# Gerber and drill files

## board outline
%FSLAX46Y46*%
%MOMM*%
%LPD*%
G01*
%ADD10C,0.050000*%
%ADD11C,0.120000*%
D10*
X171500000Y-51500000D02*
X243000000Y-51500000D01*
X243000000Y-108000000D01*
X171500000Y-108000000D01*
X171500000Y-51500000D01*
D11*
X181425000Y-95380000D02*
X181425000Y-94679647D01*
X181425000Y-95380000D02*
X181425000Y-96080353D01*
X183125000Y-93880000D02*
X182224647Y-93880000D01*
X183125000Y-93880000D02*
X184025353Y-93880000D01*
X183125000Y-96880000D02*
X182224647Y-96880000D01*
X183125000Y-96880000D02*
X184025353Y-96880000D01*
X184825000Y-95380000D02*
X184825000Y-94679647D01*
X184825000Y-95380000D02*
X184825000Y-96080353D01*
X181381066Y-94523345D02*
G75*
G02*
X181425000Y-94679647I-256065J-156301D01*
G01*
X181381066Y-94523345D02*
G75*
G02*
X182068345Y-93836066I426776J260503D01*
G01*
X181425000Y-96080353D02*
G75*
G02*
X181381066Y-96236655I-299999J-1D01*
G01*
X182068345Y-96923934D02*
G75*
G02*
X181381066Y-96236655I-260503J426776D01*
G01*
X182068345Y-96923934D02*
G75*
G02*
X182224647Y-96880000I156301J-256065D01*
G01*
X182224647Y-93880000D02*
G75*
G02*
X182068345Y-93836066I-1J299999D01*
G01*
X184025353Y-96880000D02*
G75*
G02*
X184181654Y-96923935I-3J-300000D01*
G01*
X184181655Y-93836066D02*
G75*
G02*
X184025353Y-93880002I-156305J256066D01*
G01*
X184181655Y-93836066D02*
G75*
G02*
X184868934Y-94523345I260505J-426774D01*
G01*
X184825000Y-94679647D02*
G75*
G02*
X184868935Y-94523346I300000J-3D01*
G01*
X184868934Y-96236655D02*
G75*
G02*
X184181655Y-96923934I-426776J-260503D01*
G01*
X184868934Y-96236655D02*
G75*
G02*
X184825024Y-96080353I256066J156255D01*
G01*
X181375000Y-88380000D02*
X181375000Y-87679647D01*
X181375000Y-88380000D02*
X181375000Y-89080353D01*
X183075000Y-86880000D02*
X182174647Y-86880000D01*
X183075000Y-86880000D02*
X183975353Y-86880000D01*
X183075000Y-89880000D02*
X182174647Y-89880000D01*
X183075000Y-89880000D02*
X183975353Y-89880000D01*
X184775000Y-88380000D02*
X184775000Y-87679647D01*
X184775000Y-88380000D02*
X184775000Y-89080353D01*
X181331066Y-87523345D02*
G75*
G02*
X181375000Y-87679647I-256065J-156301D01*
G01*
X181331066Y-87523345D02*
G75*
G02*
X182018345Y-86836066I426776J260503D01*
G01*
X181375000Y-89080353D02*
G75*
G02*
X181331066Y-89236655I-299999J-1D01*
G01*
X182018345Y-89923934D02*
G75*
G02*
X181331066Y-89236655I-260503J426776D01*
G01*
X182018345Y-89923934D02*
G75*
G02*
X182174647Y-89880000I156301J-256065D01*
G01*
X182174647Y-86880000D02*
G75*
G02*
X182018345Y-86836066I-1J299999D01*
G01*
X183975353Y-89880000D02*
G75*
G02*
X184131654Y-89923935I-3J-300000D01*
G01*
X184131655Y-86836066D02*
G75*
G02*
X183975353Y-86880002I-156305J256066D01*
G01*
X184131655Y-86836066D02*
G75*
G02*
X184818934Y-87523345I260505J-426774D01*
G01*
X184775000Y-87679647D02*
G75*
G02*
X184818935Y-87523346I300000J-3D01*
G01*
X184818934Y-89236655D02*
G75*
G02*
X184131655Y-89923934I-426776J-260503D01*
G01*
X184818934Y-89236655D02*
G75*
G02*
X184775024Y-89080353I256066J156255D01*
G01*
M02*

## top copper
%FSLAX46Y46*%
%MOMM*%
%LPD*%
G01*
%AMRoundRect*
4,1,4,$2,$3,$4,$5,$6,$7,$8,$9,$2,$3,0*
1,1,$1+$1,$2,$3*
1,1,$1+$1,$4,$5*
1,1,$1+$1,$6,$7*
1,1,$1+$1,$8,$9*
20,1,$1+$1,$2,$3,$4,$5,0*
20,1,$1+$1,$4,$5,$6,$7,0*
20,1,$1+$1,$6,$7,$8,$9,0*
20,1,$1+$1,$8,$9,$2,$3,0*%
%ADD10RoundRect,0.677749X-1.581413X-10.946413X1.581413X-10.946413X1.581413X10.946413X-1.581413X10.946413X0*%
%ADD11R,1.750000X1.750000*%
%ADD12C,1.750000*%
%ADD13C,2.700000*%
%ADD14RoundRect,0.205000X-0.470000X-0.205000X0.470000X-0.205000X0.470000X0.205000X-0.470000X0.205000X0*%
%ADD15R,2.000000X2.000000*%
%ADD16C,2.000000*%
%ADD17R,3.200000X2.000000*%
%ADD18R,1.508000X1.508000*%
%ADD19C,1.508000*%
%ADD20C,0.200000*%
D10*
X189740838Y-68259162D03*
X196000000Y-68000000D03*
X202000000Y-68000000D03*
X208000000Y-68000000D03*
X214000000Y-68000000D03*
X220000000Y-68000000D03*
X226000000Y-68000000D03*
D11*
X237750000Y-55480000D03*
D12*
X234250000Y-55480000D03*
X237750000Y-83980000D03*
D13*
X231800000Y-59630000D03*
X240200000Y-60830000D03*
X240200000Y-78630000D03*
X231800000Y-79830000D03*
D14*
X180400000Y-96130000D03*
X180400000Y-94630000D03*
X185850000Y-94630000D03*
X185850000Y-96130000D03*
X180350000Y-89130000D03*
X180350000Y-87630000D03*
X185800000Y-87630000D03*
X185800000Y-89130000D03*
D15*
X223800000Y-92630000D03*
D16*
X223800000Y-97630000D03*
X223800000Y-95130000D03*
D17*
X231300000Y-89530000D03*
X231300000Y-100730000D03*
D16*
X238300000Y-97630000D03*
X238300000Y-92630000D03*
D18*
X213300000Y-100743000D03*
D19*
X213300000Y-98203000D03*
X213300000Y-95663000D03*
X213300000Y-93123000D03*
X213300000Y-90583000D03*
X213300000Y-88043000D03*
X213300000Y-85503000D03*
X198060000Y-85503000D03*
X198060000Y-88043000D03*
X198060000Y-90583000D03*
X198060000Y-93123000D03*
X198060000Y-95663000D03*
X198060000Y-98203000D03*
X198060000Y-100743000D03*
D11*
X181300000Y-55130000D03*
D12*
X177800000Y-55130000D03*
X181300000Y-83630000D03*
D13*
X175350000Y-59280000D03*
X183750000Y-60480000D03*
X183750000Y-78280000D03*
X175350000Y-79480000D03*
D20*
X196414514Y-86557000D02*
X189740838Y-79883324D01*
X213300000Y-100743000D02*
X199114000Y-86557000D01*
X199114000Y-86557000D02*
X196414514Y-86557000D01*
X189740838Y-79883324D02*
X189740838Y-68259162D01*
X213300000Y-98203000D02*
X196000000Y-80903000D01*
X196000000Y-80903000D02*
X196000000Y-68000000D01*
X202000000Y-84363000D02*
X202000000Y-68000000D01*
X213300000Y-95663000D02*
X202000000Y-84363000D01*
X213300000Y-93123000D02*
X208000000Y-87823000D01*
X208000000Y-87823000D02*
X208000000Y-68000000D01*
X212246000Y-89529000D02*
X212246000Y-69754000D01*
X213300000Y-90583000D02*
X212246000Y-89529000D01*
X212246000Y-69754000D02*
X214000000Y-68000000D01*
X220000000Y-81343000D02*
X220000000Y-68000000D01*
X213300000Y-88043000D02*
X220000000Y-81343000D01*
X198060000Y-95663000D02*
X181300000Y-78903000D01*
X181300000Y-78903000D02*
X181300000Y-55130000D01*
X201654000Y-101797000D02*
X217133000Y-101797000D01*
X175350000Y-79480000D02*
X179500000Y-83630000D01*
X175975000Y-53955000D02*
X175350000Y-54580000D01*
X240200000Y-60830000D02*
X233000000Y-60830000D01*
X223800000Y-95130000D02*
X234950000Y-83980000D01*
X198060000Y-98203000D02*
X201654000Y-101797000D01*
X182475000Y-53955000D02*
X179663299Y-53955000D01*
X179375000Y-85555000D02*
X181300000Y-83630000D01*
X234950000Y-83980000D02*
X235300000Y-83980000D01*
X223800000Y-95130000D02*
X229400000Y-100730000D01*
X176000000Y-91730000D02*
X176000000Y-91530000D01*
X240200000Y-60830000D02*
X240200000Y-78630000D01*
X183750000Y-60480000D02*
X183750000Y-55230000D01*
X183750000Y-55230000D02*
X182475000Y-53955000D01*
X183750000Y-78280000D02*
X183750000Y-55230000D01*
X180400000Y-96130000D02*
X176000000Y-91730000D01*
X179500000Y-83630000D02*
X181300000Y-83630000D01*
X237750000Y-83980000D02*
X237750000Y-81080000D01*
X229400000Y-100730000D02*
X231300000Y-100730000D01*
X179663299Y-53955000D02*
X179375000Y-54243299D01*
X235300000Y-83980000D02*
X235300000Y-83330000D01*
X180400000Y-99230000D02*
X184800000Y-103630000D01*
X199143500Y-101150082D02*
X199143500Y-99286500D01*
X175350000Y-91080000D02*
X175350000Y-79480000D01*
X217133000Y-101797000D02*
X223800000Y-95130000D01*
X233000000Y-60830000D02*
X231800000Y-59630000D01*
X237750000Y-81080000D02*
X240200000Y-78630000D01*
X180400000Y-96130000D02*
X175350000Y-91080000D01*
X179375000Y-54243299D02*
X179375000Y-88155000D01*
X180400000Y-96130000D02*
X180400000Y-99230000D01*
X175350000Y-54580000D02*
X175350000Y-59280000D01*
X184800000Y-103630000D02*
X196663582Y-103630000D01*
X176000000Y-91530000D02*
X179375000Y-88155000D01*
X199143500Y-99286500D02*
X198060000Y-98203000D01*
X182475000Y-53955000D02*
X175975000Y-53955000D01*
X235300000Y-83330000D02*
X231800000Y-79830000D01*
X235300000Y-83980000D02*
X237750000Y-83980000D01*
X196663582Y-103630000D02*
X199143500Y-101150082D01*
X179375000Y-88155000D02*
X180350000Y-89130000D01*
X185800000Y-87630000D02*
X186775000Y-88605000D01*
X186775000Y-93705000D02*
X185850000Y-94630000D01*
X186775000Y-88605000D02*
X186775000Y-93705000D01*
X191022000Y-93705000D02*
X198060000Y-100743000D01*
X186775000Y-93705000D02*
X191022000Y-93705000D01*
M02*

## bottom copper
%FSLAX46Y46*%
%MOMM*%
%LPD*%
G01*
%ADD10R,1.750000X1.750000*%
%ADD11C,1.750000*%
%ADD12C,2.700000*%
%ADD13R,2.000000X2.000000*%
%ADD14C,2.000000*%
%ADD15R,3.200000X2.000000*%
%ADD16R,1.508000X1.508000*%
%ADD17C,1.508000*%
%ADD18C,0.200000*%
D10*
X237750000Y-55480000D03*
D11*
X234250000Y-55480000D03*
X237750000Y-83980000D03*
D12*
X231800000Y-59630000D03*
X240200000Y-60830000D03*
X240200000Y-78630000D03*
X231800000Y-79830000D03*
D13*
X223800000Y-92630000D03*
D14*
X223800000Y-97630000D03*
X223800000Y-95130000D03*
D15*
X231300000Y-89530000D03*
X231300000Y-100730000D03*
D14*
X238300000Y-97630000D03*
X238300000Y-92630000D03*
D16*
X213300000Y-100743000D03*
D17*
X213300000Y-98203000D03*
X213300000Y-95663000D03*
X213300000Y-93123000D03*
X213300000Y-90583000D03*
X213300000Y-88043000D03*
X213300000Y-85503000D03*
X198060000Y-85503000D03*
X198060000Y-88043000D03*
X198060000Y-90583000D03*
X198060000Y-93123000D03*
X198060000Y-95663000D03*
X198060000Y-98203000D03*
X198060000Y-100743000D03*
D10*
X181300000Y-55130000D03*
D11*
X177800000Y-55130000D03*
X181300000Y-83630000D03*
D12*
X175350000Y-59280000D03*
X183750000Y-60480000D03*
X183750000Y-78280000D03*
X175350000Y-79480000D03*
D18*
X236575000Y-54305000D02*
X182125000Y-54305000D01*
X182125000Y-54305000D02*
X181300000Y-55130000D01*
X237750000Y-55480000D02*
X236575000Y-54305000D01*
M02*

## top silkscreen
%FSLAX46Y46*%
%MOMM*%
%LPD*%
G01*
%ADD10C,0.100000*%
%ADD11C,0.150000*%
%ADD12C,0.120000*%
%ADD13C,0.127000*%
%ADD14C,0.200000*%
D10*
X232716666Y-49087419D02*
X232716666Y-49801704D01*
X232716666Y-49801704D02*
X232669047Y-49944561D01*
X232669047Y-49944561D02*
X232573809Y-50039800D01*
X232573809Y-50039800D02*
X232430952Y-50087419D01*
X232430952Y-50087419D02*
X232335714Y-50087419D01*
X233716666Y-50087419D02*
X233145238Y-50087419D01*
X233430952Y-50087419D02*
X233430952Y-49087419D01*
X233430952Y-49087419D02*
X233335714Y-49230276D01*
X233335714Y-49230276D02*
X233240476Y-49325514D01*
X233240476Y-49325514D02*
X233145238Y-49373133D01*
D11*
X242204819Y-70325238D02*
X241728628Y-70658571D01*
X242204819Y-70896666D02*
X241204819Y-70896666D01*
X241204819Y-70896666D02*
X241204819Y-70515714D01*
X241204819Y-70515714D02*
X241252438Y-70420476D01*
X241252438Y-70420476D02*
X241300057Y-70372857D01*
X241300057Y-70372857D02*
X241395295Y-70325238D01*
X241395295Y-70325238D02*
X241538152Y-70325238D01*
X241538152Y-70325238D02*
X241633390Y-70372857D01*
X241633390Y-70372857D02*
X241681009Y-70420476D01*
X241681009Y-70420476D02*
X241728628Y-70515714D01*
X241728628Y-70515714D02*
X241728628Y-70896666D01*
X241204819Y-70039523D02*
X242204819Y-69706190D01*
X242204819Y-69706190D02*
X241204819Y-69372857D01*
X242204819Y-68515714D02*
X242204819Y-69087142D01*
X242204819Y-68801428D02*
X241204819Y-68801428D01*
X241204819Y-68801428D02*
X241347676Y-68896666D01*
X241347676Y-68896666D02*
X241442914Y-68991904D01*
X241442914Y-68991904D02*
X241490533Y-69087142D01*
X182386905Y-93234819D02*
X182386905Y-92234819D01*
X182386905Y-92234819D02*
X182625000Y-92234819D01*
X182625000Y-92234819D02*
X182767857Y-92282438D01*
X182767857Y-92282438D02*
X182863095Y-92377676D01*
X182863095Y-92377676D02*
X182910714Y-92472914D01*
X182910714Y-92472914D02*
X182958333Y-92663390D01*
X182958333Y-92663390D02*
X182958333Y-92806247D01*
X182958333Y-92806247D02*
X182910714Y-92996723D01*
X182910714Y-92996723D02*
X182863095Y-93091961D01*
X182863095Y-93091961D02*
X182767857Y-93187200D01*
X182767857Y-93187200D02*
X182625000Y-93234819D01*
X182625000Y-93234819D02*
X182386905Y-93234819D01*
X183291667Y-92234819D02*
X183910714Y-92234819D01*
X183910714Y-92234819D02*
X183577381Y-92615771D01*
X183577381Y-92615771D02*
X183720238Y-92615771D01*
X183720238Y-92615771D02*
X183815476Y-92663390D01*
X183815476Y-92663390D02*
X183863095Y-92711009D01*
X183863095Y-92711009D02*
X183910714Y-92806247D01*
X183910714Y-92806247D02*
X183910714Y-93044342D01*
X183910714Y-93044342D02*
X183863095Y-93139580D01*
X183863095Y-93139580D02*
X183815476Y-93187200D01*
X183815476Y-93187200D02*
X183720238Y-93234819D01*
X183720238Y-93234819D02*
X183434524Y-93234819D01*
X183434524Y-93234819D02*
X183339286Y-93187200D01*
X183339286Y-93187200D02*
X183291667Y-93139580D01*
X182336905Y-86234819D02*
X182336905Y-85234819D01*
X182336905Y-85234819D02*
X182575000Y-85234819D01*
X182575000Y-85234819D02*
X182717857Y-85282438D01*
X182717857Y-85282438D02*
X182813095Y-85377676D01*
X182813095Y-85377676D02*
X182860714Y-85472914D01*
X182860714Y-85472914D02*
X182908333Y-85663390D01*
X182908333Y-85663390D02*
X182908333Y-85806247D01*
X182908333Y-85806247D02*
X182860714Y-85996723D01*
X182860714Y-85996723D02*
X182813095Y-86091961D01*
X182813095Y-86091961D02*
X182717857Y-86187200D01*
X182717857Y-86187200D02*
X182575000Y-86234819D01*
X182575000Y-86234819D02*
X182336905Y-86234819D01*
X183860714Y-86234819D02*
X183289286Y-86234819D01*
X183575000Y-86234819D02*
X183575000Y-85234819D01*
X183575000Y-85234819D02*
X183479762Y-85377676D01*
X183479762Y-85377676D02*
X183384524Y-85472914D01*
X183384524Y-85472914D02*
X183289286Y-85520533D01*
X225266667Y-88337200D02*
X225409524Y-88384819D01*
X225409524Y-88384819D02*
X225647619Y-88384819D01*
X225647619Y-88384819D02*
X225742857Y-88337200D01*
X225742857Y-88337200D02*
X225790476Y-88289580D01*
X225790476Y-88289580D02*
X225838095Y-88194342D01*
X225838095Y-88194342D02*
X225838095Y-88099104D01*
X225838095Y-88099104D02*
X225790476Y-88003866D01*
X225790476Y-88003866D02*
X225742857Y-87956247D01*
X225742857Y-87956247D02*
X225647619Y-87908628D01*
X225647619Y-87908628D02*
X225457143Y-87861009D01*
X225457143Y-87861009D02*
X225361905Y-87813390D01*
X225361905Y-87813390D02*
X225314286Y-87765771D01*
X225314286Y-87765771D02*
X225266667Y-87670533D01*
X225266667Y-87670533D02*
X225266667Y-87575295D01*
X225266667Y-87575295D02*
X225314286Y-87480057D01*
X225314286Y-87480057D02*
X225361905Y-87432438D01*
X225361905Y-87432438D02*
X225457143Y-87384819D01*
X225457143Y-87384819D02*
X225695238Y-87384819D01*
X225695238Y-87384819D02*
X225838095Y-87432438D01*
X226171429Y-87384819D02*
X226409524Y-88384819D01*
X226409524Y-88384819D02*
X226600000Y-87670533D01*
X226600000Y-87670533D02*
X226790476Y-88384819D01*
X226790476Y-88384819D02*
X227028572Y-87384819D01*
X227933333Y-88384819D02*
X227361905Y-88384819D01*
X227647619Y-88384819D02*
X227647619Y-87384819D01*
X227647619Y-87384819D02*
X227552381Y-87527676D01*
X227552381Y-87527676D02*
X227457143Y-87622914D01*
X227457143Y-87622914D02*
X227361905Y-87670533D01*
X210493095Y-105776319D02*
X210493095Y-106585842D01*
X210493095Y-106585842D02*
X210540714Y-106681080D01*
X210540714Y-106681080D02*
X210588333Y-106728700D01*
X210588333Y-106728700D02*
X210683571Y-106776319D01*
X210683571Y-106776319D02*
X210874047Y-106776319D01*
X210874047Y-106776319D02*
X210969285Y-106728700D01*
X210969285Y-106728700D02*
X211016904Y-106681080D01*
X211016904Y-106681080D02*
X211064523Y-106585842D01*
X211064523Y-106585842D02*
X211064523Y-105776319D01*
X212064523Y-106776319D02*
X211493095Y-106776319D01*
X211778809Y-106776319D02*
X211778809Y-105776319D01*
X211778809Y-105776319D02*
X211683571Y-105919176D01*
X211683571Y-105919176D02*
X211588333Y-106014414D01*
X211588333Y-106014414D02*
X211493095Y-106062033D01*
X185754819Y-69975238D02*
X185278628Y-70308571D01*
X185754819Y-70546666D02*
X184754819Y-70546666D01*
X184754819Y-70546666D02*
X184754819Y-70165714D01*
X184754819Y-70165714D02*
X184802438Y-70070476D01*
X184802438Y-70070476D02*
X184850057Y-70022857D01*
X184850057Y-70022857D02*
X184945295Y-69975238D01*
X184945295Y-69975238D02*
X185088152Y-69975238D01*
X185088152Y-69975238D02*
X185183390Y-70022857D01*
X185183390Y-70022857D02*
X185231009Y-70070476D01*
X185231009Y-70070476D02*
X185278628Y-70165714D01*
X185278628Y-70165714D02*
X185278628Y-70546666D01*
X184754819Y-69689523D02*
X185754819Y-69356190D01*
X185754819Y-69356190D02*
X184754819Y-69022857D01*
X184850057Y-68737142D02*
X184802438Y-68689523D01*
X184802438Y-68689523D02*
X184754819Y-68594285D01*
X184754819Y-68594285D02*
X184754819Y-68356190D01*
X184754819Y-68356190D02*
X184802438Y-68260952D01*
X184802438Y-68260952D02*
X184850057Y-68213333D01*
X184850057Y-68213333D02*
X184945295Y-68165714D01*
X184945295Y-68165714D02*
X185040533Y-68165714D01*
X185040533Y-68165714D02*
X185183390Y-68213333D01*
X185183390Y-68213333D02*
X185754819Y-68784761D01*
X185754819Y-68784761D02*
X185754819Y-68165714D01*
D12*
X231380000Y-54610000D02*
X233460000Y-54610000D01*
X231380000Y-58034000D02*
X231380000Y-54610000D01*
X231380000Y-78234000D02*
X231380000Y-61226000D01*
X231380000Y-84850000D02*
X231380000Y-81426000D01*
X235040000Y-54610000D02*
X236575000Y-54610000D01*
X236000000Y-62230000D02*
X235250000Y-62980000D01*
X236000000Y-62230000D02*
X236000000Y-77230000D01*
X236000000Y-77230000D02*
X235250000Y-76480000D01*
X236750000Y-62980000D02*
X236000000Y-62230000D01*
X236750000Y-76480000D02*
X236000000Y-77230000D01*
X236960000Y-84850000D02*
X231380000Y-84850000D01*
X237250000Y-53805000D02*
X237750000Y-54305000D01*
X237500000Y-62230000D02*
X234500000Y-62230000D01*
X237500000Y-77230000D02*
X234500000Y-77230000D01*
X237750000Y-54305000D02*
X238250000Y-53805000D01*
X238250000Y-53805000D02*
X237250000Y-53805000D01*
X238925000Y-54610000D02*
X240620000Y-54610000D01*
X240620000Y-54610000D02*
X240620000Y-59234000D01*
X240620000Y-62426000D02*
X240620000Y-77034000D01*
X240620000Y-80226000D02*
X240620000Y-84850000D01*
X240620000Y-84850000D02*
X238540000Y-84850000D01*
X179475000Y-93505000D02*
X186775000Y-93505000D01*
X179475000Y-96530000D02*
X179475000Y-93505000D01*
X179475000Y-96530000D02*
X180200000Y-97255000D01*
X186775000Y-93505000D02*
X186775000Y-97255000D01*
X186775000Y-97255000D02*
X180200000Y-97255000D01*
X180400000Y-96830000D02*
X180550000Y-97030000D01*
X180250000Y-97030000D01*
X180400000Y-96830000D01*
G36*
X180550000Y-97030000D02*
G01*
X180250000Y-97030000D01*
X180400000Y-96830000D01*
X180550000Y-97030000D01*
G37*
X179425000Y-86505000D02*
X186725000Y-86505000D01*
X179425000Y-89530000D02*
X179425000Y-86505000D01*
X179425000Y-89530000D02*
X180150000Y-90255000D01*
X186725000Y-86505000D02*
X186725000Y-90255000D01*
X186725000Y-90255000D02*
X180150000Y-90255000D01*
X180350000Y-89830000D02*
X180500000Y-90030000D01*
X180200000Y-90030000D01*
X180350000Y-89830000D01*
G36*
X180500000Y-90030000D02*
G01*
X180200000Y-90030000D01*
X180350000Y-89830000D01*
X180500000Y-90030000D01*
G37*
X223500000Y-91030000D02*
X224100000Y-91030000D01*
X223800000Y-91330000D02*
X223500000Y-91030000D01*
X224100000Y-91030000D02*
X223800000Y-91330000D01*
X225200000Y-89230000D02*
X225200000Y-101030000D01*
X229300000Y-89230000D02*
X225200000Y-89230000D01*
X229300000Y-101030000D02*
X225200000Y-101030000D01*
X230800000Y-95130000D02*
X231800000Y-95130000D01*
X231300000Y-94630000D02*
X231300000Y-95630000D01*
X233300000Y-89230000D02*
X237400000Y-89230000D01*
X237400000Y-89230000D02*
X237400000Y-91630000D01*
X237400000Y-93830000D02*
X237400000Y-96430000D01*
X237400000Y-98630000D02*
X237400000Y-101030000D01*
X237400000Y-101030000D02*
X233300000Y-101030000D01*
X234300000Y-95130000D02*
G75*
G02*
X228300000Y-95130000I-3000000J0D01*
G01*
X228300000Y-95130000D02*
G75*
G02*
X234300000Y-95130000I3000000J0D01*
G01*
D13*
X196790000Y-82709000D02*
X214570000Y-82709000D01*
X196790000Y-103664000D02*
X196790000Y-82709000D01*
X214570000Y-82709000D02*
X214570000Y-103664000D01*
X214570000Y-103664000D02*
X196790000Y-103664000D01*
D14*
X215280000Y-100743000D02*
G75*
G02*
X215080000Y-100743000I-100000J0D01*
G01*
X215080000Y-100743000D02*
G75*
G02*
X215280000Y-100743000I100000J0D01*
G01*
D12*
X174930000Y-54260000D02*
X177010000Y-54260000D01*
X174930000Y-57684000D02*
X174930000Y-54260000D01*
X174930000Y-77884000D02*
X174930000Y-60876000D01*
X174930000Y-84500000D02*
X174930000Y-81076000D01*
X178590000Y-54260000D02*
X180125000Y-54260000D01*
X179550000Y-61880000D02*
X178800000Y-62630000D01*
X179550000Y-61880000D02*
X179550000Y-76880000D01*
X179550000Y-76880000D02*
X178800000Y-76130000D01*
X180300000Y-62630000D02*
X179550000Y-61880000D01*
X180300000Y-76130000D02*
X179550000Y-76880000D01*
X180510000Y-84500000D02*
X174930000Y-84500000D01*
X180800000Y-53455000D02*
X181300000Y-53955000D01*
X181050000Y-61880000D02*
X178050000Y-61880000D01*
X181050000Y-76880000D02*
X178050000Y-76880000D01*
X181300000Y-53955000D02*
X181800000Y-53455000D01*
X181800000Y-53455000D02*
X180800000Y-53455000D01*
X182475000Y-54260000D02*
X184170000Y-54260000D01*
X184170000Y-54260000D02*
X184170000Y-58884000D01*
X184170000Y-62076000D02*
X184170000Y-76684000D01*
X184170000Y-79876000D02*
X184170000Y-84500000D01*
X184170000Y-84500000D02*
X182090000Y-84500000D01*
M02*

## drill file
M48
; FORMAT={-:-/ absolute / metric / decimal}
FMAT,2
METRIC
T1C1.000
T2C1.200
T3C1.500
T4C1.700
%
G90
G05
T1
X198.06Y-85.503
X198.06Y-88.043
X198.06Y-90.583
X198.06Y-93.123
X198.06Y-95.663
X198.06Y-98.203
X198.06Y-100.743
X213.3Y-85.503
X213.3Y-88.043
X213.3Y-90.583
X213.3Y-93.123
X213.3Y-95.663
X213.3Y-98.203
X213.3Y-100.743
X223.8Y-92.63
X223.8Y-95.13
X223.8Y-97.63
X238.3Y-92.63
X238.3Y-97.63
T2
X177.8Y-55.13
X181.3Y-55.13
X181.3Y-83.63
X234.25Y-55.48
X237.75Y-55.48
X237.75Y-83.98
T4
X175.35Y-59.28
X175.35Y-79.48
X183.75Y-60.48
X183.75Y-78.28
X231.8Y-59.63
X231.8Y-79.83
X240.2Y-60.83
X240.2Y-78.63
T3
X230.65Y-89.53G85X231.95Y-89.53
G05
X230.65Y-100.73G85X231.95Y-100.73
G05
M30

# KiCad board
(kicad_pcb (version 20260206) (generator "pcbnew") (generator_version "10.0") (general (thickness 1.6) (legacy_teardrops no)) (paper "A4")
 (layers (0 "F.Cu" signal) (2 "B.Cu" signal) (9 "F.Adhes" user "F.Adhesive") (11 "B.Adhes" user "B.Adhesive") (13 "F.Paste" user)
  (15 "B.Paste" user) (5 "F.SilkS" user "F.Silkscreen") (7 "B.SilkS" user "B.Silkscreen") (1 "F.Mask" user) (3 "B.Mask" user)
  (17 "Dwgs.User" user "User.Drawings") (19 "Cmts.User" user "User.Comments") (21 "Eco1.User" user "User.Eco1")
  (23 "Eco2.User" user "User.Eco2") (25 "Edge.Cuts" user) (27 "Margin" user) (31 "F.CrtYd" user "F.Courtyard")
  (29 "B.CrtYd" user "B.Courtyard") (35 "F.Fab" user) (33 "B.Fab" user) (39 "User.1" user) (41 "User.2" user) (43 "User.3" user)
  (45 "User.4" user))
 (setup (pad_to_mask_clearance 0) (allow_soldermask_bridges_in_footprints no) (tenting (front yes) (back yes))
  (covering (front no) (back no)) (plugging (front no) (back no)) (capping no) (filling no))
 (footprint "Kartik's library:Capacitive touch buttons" (layer "F.Cu") (at 204 54)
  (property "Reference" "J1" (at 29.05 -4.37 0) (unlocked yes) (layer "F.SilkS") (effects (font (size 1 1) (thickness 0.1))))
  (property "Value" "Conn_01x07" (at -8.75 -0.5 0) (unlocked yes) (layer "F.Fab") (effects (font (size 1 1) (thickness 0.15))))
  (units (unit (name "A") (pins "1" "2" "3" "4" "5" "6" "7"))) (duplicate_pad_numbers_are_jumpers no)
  (pad "1" smd roundrect (at -14.259162 14.259162) (size 4.518324 23.248324) (layers "F.Cu" "F.Mask" "F.Paste") (roundrect_rratio 0.15)
   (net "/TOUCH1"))
  (pad "2" smd roundrect (at -8 14) (size 4.518324 23.248324) (layers "F.Cu" "F.Mask" "F.Paste") (roundrect_rratio 0.15) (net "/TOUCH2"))
  (pad "3" smd roundrect (at -2 14) (size 4.518324 23.248324) (layers "F.Cu" "F.Mask" "F.Paste") (roundrect_rratio 0.15) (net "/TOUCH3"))
  (pad "4" smd roundrect (at 4 14) (size 4.518324 23.248324) (layers "F.Cu" "F.Mask" "F.Paste") (roundrect_rratio 0.15) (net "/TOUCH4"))
  (pad "5" smd roundrect (at 10 14) (size 4.518324 23.248324) (layers "F.Cu" "F.Mask" "F.Paste") (roundrect_rratio 0.15) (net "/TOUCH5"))
  (pad "6" smd roundrect (at 16 14) (size 4.518324 23.248324) (layers "F.Cu" "F.Mask" "F.Paste") (roundrect_rratio 0.15) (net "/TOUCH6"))
  (pad "7" smd roundrect (at 22 14) (size 4.518324 23.248324) (layers "F.Cu" "F.Mask" "F.Paste") (roundrect_rratio 0.15) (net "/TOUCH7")))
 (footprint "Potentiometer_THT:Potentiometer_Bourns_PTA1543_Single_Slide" (layer "F.Cu") (at 237.75 55.48 -90)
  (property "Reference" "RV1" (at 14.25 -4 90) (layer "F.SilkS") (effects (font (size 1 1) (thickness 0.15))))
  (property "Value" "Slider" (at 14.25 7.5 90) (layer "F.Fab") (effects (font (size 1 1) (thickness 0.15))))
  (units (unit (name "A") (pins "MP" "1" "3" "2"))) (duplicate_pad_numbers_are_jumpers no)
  (fp_line (start -0.87 6.37) (end -0.87 4.29) (stroke (width 0.12) (type solid)) (layer "F.SilkS"))
  (fp_line (start 2.554 6.37) (end -0.87 6.37) (stroke (width 0.12) (type solid)) (layer "F.SilkS"))
  (fp_line (start 22.754 6.37) (end 5.746 6.37) (stroke (width 0.12) (type solid)) (layer "F.SilkS"))
  (fp_line (start 29.37 6.37) (end 25.946 6.37) (stroke (width 0.12) (type solid)) (layer "F.SilkS"))
  (fp_line (start -0.87 2.71) (end -0.87 1.175) (stroke (width 0.12) (type solid)) (layer "F.SilkS"))
  (fp_line (start 6.75 1.75) (end 7.5 2.5) (stroke (width 0.12) (type solid)) (layer "F.SilkS"))
  (fp_line (start 6.75 1.75) (end 21.75 1.75) (stroke (width 0.12) (type solid)) (layer "F.SilkS"))
  (fp_line (start 21.75 1.75) (end 21 2.5) (stroke (width 0.12) (type solid)) (layer "F.SilkS"))
  (fp_line (start 7.5 1) (end 6.75 1.75) (stroke (width 0.12) (type solid)) (layer "F.SilkS"))
  (fp_line (start 21 1) (end 21.75 1.75) (stroke (width 0.12) (type solid)) (layer "F.SilkS"))
  (fp_line (start 29.37 0.79) (end 29.37 6.37) (stroke (width 0.12) (type solid)) (layer "F.SilkS"))
  (fp_line (start -1.675 0.5) (end -1.175 0) (stroke (width 0.12) (type solid)) (layer "F.SilkS"))
  (fp_line (start 6.75 0.25) (end 6.75 3.25) (stroke (width 0.12) (type solid)) (layer "F.SilkS"))
  (fp_line (start 21.75 0.25) (end 21.75 3.25) (stroke (width 0.12) (type solid)) (layer "F.SilkS"))
  (fp_line (start -1.175 0) (end -1.675 -0.5) (stroke (width 0.12) (type solid)) (layer "F.SilkS"))
  (fp_line (start -1.675 -0.5) (end -1.675 0.5) (stroke (width 0.12) (type solid)) (layer "F.SilkS"))
  (fp_line (start -0.87 -1.175) (end -0.87 -2.87) (stroke (width 0.12) (type solid)) (layer "F.SilkS"))
  (fp_line (start -0.87 -2.87) (end 3.754 -2.87) (stroke (width 0.12) (type solid)) (layer "F.SilkS"))
  (fp_line (start 6.946 -2.87) (end 21.554 -2.87) (stroke (width 0.12) (type solid)) (layer "F.SilkS"))
  (fp_line (start 24.746 -2.87) (end 29.37 -2.87) (stroke (width 0.12) (type solid)) (layer "F.SilkS"))
  (fp_line (start 29.37 -2.87) (end 29.37 -0.79) (stroke (width 0.12) (type solid)) (layer "F.SilkS"))
  (pad "1" thru_hole rect (at 0 0 270) (size 1.75 1.75) (drill 1.2) (layers "*.Cu" "*.Mask") (remove_unused_layers no) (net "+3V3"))
  (pad "2" thru_hole circle (at 0 3.5 270) (size 1.75 1.75) (drill 1.2) (layers "*.Cu" "*.Mask") (remove_unused_layers no) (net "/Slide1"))
  (pad "3" thru_hole circle (at 28.5 0 270) (size 1.75 1.75) (drill 1.2) (layers "*.Cu" "*.Mask") (remove_unused_layers no) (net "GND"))
  (pad "MP" thru_hole circle (at 4.15 5.95 270) (size 2.7 2.7) (drill 1.7) (layers "*.Cu" "*.Mask") (remove_unused_layers no) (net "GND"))
  (pad "MP" thru_hole circle (at 5.35 -2.45 270) (size 2.7 2.7) (drill 1.7) (layers "*.Cu" "*.Mask") (remove_unused_layers no) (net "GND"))
  (pad "MP" thru_hole circle (at 23.15 -2.45 270) (size 2.7 2.7) (drill 1.7) (layers "*.Cu" "*.Mask") (remove_unused_layers no) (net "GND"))
  (pad "MP" thru_hole circle (at 24.35 5.95 270) (size 2.7 2.7) (drill 1.7) (layers "*.Cu" "*.Mask") (remove_unused_layers no) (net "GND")))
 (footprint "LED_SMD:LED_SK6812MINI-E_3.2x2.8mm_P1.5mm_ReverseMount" (layer "F.Cu") (at 183.125 95.38)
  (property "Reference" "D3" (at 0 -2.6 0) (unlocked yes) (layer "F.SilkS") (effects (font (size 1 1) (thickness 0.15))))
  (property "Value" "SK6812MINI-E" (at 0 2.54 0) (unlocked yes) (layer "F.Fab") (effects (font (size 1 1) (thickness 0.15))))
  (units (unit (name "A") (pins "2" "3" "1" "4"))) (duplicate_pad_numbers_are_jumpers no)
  (fp_line (start -3.65 -1.875) (end 3.65 -1.875) (stroke (width 0.12) (type solid)) (layer "F.SilkS"))
  (fp_line (start -3.65 1.15) (end -3.65 -1.875) (stroke (width 0.12) (type solid)) (layer "F.SilkS"))
  (fp_line (start -3.65 1.15) (end -2.925 1.875) (stroke (width 0.12) (type solid)) (layer "F.SilkS"))
  (fp_line (start 3.65 -1.875) (end 3.65 1.875) (stroke (width 0.12) (type solid)) (layer "F.SilkS"))
  (fp_line (start 3.65 1.875) (end -2.925 1.875) (stroke (width 0.12) (type solid)) (layer "F.SilkS"))
  (fp_poly (pts (xy -2.725 1.45) (xy -2.575 1.65) (xy -2.875 1.65)) (stroke (width 0.12) (type solid)) (fill yes) (layer "F.SilkS"))
  (fp_line (start -1.7 0) (end -1.7 -0.700353) (stroke (width 0.12) (type solid)) (layer "Edge.Cuts"))
  (fp_line (start -1.7 0) (end -1.7 0.700353) (stroke (width 0.12) (type solid)) (layer "Edge.Cuts"))
  (fp_line (start 0 -1.5) (end -0.900353 -1.5) (stroke (width 0.12) (type solid)) (layer "Edge.Cuts"))
  (fp_line (start 0 -1.5) (end 0.900353 -1.5) (stroke (width 0.12) (type solid)) (layer "Edge.Cuts"))
  (fp_line (start 0 1.5) (end -0.900353 1.5) (stroke (width 0.12) (type solid)) (layer "Edge.Cuts"))
  (fp_line (start 0 1.5) (end 0.900353 1.5) (stroke (width 0.12) (type solid)) (layer "Edge.Cuts"))
  (fp_line (start 1.7 0) (end 1.7 -0.700353) (stroke (width 0.12) (type solid)) (layer "Edge.Cuts"))
  (fp_line (start 1.7 0) (end 1.7 0.700353) (stroke (width 0.12) (type solid)) (layer "Edge.Cuts"))
  (fp_arc (start -1.743934 -0.856655) (mid -1.711192 -0.781532) (end -1.7 -0.700353) (stroke (width 0.12) (type solid)) (layer "Edge.Cuts"))
  (fp_arc (start -1.743934 -0.856655) (mid -1.670711 -1.470711) (end -1.056655 -1.543934) (stroke (width 0.12) (type solid))
   (layer "Edge.Cuts"))
  (fp_arc (start -1.7 0.700353) (mid -1.711192 0.781532) (end -1.743934 0.856655) (stroke (width 0.12) (type solid)) (layer "Edge.Cuts"))
  (fp_arc (start -1.056655 1.543934) (mid -1.670711 1.470711) (end -1.743934 0.856655) (stroke (width 0.12) (type solid))
   (layer "Edge.Cuts"))
  (fp_arc (start -1.056655 1.543934) (mid -0.981532 1.511192) (end -0.900353 1.5) (stroke (width 0.12) (type solid)) (layer "Edge.Cuts"))
  (fp_arc (start -0.900353 -1.5) (mid -0.981532 -1.511192) (end -1.056655 -1.543934) (stroke (width 0.12) (type solid)) (layer "Edge.Cuts"))
  (fp_arc (start 0.900353 1.5) (mid 0.981532 1.511192) (end 1.056655 1.543934) (stroke (width 0.12) (type solid)) (layer "Edge.Cuts"))
  (fp_arc (start 1.056655 -1.543934) (mid 0.981532 -1.511192) (end 0.900353 -1.5) (stroke (width 0.12) (type solid)) (layer "Edge.Cuts"))
  (fp_arc (start 1.056655 -1.543934) (mid 1.670711 -1.470711) (end 1.743934 -0.856655) (stroke (width 0.12) (type solid))
   (layer "Edge.Cuts"))
  (fp_arc (start 1.7 -0.700353) (mid 1.711192 -0.781532) (end 1.743934 -0.856655) (stroke (width 0.12) (type solid)) (layer "Edge.Cuts"))
  (fp_arc (start 1.743934 0.856655) (mid 1.670711 1.470711) (end 1.056655 1.543934) (stroke (width 0.12) (type solid)) (layer "Edge.Cuts"))
  (fp_arc (start 1.743934 0.856655) (mid 1.711192 0.781532) (end 1.7 0.700353) (stroke (width 0.12) (type solid)) (layer "Edge.Cuts"))
  (pad "1" smd roundrect (at -2.725 0.75) (size 1.35 0.82) (layers "F.Cu" "F.Mask" "F.Paste") (roundrect_rratio 0.25) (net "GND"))
  (pad "2" smd roundrect (at -2.725 -0.75) (size 1.35 0.82) (layers "F.Cu" "F.Mask" "F.Paste") (roundrect_rratio 0.25) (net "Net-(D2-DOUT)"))
  (pad "3" smd roundrect (at 2.725 -0.75) (size 1.35 0.82) (layers "F.Cu" "F.Mask" "F.Paste") (roundrect_rratio 0.25) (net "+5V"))
  (pad "4" smd roundrect (at 2.725 0.75) (size 1.35 0.82) (layers "F.Cu" "F.Mask" "F.Paste") (roundrect_rratio 0.25)
   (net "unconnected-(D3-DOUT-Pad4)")))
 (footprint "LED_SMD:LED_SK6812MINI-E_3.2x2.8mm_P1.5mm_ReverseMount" (layer "F.Cu") (at 183.075 88.38)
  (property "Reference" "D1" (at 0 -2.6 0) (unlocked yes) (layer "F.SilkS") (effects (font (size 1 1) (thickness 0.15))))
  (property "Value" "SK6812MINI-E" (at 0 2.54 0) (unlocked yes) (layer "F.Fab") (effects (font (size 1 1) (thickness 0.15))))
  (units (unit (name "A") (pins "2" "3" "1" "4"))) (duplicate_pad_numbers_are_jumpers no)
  (fp_line (start -3.65 -1.875) (end 3.65 -1.875) (stroke (width 0.12) (type solid)) (layer "F.SilkS"))
  (fp_line (start -3.65 1.15) (end -3.65 -1.875) (stroke (width 0.12) (type solid)) (layer "F.SilkS"))
  (fp_line (start -3.65 1.15) (end -2.925 1.875) (stroke (width 0.12) (type solid)) (layer "F.SilkS"))
  (fp_line (start 3.65 -1.875) (end 3.65 1.875) (stroke (width 0.12) (type solid)) (layer "F.SilkS"))
  (fp_line (start 3.65 1.875) (end -2.925 1.875) (stroke (width 0.12) (type solid)) (layer "F.SilkS"))
  (fp_poly (pts (xy -2.725 1.45) (xy -2.575 1.65) (xy -2.875 1.65)) (stroke (width 0.12) (type solid)) (fill yes) (layer "F.SilkS"))
  (fp_line (start -1.7 0) (end -1.7 -0.700353) (stroke (width 0.12) (type solid)) (layer "Edge.Cuts"))
  (fp_line (start -1.7 0) (end -1.7 0.700353) (stroke (width 0.12) (type solid)) (layer "Edge.Cuts"))
  (fp_line (start 0 -1.5) (end -0.900353 -1.5) (stroke (width 0.12) (type solid)) (layer "Edge.Cuts"))
  (fp_line (start 0 -1.5) (end 0.900353 -1.5) (stroke (width 0.12) (type solid)) (layer "Edge.Cuts"))
  (fp_line (start 0 1.5) (end -0.900353 1.5) (stroke (width 0.12) (type solid)) (layer "Edge.Cuts"))
  (fp_line (start 0 1.5) (end 0.900353 1.5) (stroke (width 0.12) (type solid)) (layer "Edge.Cuts"))
  (fp_line (start 1.7 0) (end 1.7 -0.700353) (stroke (width 0.12) (type solid)) (layer "Edge.Cuts"))
  (fp_line (start 1.7 0) (end 1.7 0.700353) (stroke (width 0.12) (type solid)) (layer "Edge.Cuts"))
  (fp_arc (start -1.743934 -0.856655) (mid -1.711192 -0.781532) (end -1.7 -0.700353) (stroke (width 0.12) (type solid)) (layer "Edge.Cuts"))
  (fp_arc (start -1.743934 -0.856655) (mid -1.670711 -1.470711) (end -1.056655 -1.543934) (stroke (width 0.12) (type solid))
   (layer "Edge.Cuts"))
  (fp_arc (start -1.7 0.700353) (mid -1.711192 0.781532) (end -1.743934 0.856655) (stroke (width 0.12) (type solid)) (layer "Edge.Cuts"))
  (fp_arc (start -1.056655 1.543934) (mid -1.670711 1.470711) (end -1.743934 0.856655) (stroke (width 0.12) (type solid))
   (layer "Edge.Cuts"))
  (fp_arc (start -1.056655 1.543934) (mid -0.981532 1.511192) (end -0.900353 1.5) (stroke (width 0.12) (type solid)) (layer "Edge.Cuts"))
  (fp_arc (start -0.900353 -1.5) (mid -0.981532 -1.511192) (end -1.056655 -1.543934) (stroke (width 0.12) (type solid)) (layer "Edge.Cuts"))
  (fp_arc (start 0.900353 1.5) (mid 0.981532 1.511192) (end 1.056655 1.543934) (stroke (width 0.12) (type solid)) (layer "Edge.Cuts"))
  (fp_arc (start 1.056655 -1.543934) (mid 0.981532 -1.511192) (end 0.900353 -1.5) (stroke (width 0.12) (type solid)) (layer "Edge.Cuts"))
  (fp_arc (start 1.056655 -1.543934) (mid 1.670711 -1.470711) (end 1.743934 -0.856655) (stroke (width 0.12) (type solid))
   (layer "Edge.Cuts"))
  (fp_arc (start 1.7 -0.700353) (mid 1.711192 -0.781532) (end 1.743934 -0.856655) (stroke (width 0.12) (type solid)) (layer "Edge.Cuts"))
  (fp_arc (start 1.743934 0.856655) (mid 1.670711 1.470711) (end 1.056655 1.543934) (stroke (width 0.12) (type solid)) (layer "Edge.Cuts"))
  (fp_arc (start 1.743934 0.856655) (mid 1.711192 0.781532) (end 1.7 0.700353) (stroke (width 0.12) (type solid)) (layer "Edge.Cuts"))
  (pad "1" smd roundrect (at -2.725 0.75) (size 1.35 0.82) (layers "F.Cu" "F.Mask" "F.Paste") (roundrect_rratio 0.25) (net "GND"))
  (pad "2" smd roundrect (at -2.725 -0.75) (size 1.35 0.82) (layers "F.Cu" "F.Mask" "F.Paste") (roundrect_rratio 0.25) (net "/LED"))
  (pad "3" smd roundrect (at 2.725 -0.75) (size 1.35 0.82) (layers "F.Cu" "F.Mask" "F.Paste") (roundrect_rratio 0.25) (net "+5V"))
  (pad "4" smd roundrect (at 2.725 0.75) (size 1.35 0.82) (layers "F.Cu" "F.Mask" "F.Paste") (roundrect_rratio 0.25) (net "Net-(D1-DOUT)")))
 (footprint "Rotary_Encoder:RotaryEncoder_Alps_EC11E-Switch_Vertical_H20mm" (layer "F.Cu") (at 223.8 92.63)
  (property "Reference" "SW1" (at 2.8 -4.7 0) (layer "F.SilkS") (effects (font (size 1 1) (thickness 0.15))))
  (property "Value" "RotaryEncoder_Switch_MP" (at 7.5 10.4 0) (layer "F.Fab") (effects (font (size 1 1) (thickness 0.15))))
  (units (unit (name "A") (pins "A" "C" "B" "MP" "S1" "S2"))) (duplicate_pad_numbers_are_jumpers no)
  (fp_line (start -0.3 -1.6) (end 0.3 -1.6) (stroke (width 0.12) (type solid)) (layer "F.SilkS"))
  (fp_line (start 0 -1.3) (end -0.3 -1.6) (stroke (width 0.12) (type solid)) (layer "F.SilkS"))
  (fp_line (start 0.3 -1.6) (end 0 -1.3) (stroke (width 0.12) (type solid)) (layer "F.SilkS"))
  (fp_line (start 1.4 -3.4) (end 1.4 8.4) (stroke (width 0.12) (type solid)) (layer "F.SilkS"))
  (fp_line (start 5.5 -3.4) (end 1.4 -3.4) (stroke (width 0.12) (type solid)) (layer "F.SilkS"))
  (fp_line (start 5.5 8.4) (end 1.4 8.4) (stroke (width 0.12) (type solid)) (layer "F.SilkS"))
  (fp_line (start 7 2.5) (end 8 2.5) (stroke (width 0.12) (type solid)) (layer "F.SilkS"))
  (fp_line (start 7.5 2) (end 7.5 3) (stroke (width 0.12) (type solid)) (layer "F.SilkS"))
  (fp_line (start 9.5 -3.4) (end 13.6 -3.4) (stroke (width 0.12) (type solid)) (layer "F.SilkS"))
  (fp_line (start 13.6 -3.4) (end 13.6 -1) (stroke (width 0.12) (type solid)) (layer "F.SilkS"))
  (fp_line (start 13.6 1.2) (end 13.6 3.8) (stroke (width 0.12) (type solid)) (layer "F.SilkS"))
  (fp_line (start 13.6 6) (end 13.6 8.4) (stroke (width 0.12) (type solid)) (layer "F.SilkS"))
  (fp_line (start 13.6 8.4) (end 9.5 8.4) (stroke (width 0.12) (type solid)) (layer "F.SilkS"))
  (fp_circle (center 7.5 2.5) (end 10.5 2.5) (stroke (width 0.12) (type solid)) (fill no) (layer "F.SilkS"))
  (pad "A" thru_hole rect (at 0 0) (size 2 2) (drill 1) (layers "*.Cu" "*.Mask") (remove_unused_layers no) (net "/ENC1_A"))
  (pad "B" thru_hole circle (at 0 5) (size 2 2) (drill 1) (layers "*.Cu" "*.Mask") (remove_unused_layers no) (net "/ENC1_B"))
  (pad "C" thru_hole circle (at 0 2.5) (size 2 2) (drill 1) (layers "*.Cu" "*.Mask") (remove_unused_layers no) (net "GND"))
  (pad "MP" thru_hole rect (at 7.5 -3.1) (size 3.2 2) (drill oval 2.8 1.5) (layers "*.Cu" "*.Mask") (remove_unused_layers no) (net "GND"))
  (pad "MP" thru_hole rect (at 7.5 8.1) (size 3.2 2) (drill oval 2.8 1.5) (layers "*.Cu" "*.Mask") (remove_unused_layers no) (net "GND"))
  (pad "S1" thru_hole circle (at 14.5 5) (size 2 2) (drill 1) (layers "*.Cu" "*.Mask") (remove_unused_layers no)
   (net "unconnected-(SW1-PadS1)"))
  (pad "S2" thru_hole circle (at 14.5 0) (size 2 2) (drill 1) (layers "*.Cu" "*.Mask") (remove_unused_layers no)
   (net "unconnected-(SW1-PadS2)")))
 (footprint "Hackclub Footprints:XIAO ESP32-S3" (layer "F.Cu") (at 205.68 93.1865 180)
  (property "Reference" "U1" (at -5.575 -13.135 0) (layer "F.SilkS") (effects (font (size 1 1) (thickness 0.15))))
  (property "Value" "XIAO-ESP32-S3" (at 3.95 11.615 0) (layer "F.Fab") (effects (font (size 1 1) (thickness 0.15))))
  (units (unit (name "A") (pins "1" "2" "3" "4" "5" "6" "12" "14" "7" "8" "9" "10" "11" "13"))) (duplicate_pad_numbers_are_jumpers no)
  (fp_line (start 8.89 10.4775) (end -8.89 10.4775) (stroke (width 0.127) (type solid)) (layer "F.SilkS"))
  (fp_line (start 8.89 -10.4775) (end 8.89 10.4775) (stroke (width 0.127) (type solid)) (layer "F.SilkS"))
  (fp_line (start -8.89 10.4775) (end -8.89 -10.4775) (stroke (width 0.127) (type solid)) (layer "F.SilkS"))
  (fp_line (start -8.89 -10.4775) (end 8.89 -10.4775) (stroke (width 0.127) (type solid)) (layer "F.SilkS"))
  (fp_circle (center -9.5 -7.5565) (end -9.4 -7.5565) (stroke (width 0.2) (type solid)) (fill no) (layer "F.SilkS"))
  (pad "1" thru_hole rect (at -7.62 -7.5565 180) (size 1.508 1.508) (drill 1) (layers "*.Cu" "*.Mask") (remove_unused_layers no)
   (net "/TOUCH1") (solder_mask_margin 0.102))
  (pad "2" thru_hole circle (at -7.62 -5.0165 180) (size 1.508 1.508) (drill 1) (layers "*.Cu" "*.Mask") (remove_unused_layers no)
   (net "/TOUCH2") (solder_mask_margin 0.102))
  (pad "3" thru_hole circle (at -7.62 -2.4765 180) (size 1.508 1.508) (drill 1) (layers "*.Cu" "*.Mask") (remove_unused_layers no)
   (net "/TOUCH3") (solder_mask_margin 0.102))
  (pad "4" thru_hole circle (at -7.62 0.0635 180) (size 1.508 1.508) (drill 1) (layers "*.Cu" "*.Mask") (remove_unused_layers no)
   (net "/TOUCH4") (solder_mask_margin 0.102))
  (pad "5" thru_hole circle (at -7.62 2.6035 180) (size 1.508 1.508) (drill 1) (layers "*.Cu" "*.Mask") (remove_unused_layers no)
   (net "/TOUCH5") (solder_mask_margin 0.102))
  (pad "6" thru_hole circle (at -7.62 5.1435 180) (size 1.508 1.508) (drill 1) (layers "*.Cu" "*.Mask") (remove_unused_layers no)
   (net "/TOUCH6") (solder_mask_margin 0.102))
  (pad "7" thru_hole circle (at -7.62 7.6835 180) (size 1.508 1.508) (drill 1) (layers "*.Cu" "*.Mask") (remove_unused_layers no)
   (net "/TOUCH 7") (solder_mask_margin 0.102))
  (pad "8" thru_hole circle (at 7.62 7.6835 180) (size 1.508 1.508) (drill 1) (layers "*.Cu" "*.Mask") (remove_unused_layers no)
   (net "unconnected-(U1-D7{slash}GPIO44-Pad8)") (solder_mask_margin 0.102))
  (pad "9" thru_hole circle (at 7.62 5.1435 180) (size 1.508 1.508) (drill 1) (layers "*.Cu" "*.Mask") (remove_unused_layers no)
   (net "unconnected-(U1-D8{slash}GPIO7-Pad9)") (solder_mask_margin 0.102))
  (pad "10" thru_hole circle (at 7.62 2.6035 180) (size 1.508 1.508) (drill 1) (layers "*.Cu" "*.Mask") (remove_unused_layers no)
   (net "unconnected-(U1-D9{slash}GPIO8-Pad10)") (solder_mask_margin 0.102))
  (pad "11" thru_hole circle (at 7.62 0.0635 180) (size 1.508 1.508) (drill 1) (layers "*.Cu" "*.Mask") (remove_unused_layers no)
   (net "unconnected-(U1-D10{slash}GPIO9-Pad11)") (solder_mask_margin 0.102))
  (pad "12" thru_hole circle (at 7.62 -2.4765 180) (size 1.508 1.508) (drill 1) (layers "*.Cu" "*.Mask") (remove_unused_layers no)
   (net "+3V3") (solder_mask_margin 0.102))
  (pad "13" thru_hole circle (at 7.62 -5.0165 180) (size 1.508 1.508) (drill 1) (layers "*.Cu" "*.Mask") (remove_unused_layers no)
   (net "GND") (solder_mask_margin 0.102))
  (pad "14" thru_hole circle (at 7.62 -7.5565 180) (size 1.508 1.508) (drill 1) (layers "*.Cu" "*.Mask") (remove_unused_layers no)
   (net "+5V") (solder_mask_margin 0.102)))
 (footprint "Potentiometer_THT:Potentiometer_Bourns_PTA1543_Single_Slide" (layer "F.Cu") (at 181.3 55.13 -90)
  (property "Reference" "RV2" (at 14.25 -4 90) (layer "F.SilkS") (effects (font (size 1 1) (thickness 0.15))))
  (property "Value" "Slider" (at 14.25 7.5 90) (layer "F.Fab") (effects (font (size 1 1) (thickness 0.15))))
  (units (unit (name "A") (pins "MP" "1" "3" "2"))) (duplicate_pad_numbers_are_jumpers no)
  (fp_line (start -0.87 6.37) (end -0.87 4.29) (stroke (width 0.12) (type solid)) (layer "F.SilkS"))
  (fp_line (start 2.554 6.37) (end -0.87 6.37) (stroke (width 0.12) (type solid)) (layer "F.SilkS"))
  (fp_line (start 22.754 6.37) (end 5.746 6.37) (stroke (width 0.12) (type solid)) (layer "F.SilkS"))
  (fp_line (start 29.37 6.37) (end 25.946 6.37) (stroke (width 0.12) (type solid)) (layer "F.SilkS"))
  (fp_line (start -0.87 2.71) (end -0.87 1.175) (stroke (width 0.12) (type solid)) (layer "F.SilkS"))
  (fp_line (start 6.75 1.75) (end 7.5 2.5) (stroke (width 0.12) (type solid)) (layer "F.SilkS"))
  (fp_line (start 6.75 1.75) (end 21.75 1.75) (stroke (width 0.12) (type solid)) (layer "F.SilkS"))
  (fp_line (start 21.75 1.75) (end 21 2.5) (stroke (width 0.12) (type solid)) (layer "F.SilkS"))
  (fp_line (start 7.5 1) (end 6.75 1.75) (stroke (width 0.12) (type solid)) (layer "F.SilkS"))
  (fp_line (start 21 1) (end 21.75 1.75) (stroke (width 0.12) (type solid)) (layer "F.SilkS"))
  (fp_line (start 29.37 0.79) (end 29.37 6.37) (stroke (width 0.12) (type solid)) (layer "F.SilkS"))
  (fp_line (start -1.675 0.5) (end -1.175 0) (stroke (width 0.12) (type solid)) (layer "F.SilkS"))
  (fp_line (start 6.75 0.25) (end 6.75 3.25) (stroke (width 0.12) (type solid)) (layer "F.SilkS"))
  (fp_line (start 21.75 0.25) (end 21.75 3.25) (stroke (width 0.12) (type solid)) (layer "F.SilkS"))
  (fp_line (start -1.175 0) (end -1.675 -0.5) (stroke (width 0.12) (type solid)) (layer "F.SilkS"))
  (fp_line (start -1.675 -0.5) (end -1.675 0.5) (stroke (width 0.12) (type solid)) (layer "F.SilkS"))
  (fp_line (start -0.87 -1.175) (end -0.87 -2.87) (stroke (width 0.12) (type solid)) (layer "F.SilkS"))
  (fp_line (start -0.87 -2.87) (end 3.754 -2.87) (stroke (width 0.12) (type solid)) (layer "F.SilkS"))
  (fp_line (start 6.946 -2.87) (end 21.554 -2.87) (stroke (width 0.12) (type solid)) (layer "F.SilkS"))
  (fp_line (start 24.746 -2.87) (end 29.37 -2.87) (stroke (width 0.12) (type solid)) (layer "F.SilkS"))
  (fp_line (start 29.37 -2.87) (end 29.37 -0.79) (stroke (width 0.12) (type solid)) (layer "F.SilkS"))
  (pad "1" thru_hole rect (at 0 0 270) (size 1.75 1.75) (drill 1.2) (layers "*.Cu" "*.Mask") (remove_unused_layers no) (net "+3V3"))
  (pad "2" thru_hole circle (at 0 3.5 270) (size 1.75 1.75) (drill 1.2) (layers "*.Cu" "*.Mask") (remove_unused_layers no) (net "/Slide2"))
  (pad "3" thru_hole circle (at 28.5 0 270) (size 1.75 1.75) (drill 1.2) (layers "*.Cu" "*.Mask") (remove_unused_layers no) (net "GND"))
  (pad "MP" thru_hole circle (at 4.15 5.95 270) (size 2.7 2.7) (drill 1.7) (layers "*.Cu" "*.Mask") (remove_unused_layers no) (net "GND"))
  (pad "MP" thru_hole circle (at 5.35 -2.45 270) (size 2.7 2.7) (drill 1.7) (layers "*.Cu" "*.Mask") (remove_unused_layers no) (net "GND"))
  (pad "MP" thru_hole circle (at 23.15 -2.45 270) (size 2.7 2.7) (drill 1.7) (layers "*.Cu" "*.Mask") (remove_unused_layers no) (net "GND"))
  (pad "MP" thru_hole circle (at 24.35 5.95 270) (size 2.7 2.7) (drill 1.7) (layers "*.Cu" "*.Mask") (remove_unused_layers no) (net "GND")))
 (gr_rect (start 171.5 51.5) (end 243 108) (stroke (width 0.05) (type default)) (fill no) (layer "Edge.Cuts"))
 (segment (start 196.414514 86.557) (end 189.740838 79.883324) (width 0.2) (layer "F.Cu") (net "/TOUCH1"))
 (segment (start 213.3 100.743) (end 199.114 86.557) (width 0.2) (layer "F.Cu") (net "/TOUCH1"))
 (segment (start 199.114 86.557) (end 196.414514 86.557) (width 0.2) (layer "F.Cu") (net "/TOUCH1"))
 (segment (start 189.740838 79.883324) (end 189.740838 68.259162) (width 0.2) (layer "F.Cu") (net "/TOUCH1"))
 (segment (start 213.3 98.203) (end 196 80.903) (width 0.2) (layer "F.Cu") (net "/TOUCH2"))
 (segment (start 196 80.903) (end 196 68) (width 0.2) (layer "F.Cu") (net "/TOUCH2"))
 (segment (start 202 84.363) (end 202 68) (width 0.2) (layer "F.Cu") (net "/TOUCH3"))
 (segment (start 213.3 95.663) (end 202 84.363) (width 0.2) (layer "F.Cu") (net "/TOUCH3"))
 (segment (start 213.3 93.123) (end 208 87.823) (width 0.2) (layer "F.Cu") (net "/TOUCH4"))
 (segment (start 208 87.823) (end 208 68) (width 0.2) (layer "F.Cu") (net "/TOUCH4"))
 (segment (start 212.246 89.529) (end 212.246 69.754) (width 0.2) (layer "F.Cu") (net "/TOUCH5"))
 (segment (start 213.3 90.583) (end 212.246 89.529) (width 0.2) (layer "F.Cu") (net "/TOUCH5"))
 (segment (start 212.246 69.754) (end 214 68) (width 0.2) (layer "F.Cu") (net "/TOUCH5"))
 (segment (start 220 81.343) (end 220 68) (width 0.2) (layer "F.Cu") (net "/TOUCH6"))
 (segment (start 213.3 88.043) (end 220 81.343) (width 0.2) (layer "F.Cu") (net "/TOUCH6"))
 (segment (start 198.06 95.663) (end 181.3 78.903) (width 0.2) (layer "F.Cu") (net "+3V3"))
 (segment (start 181.3 78.903) (end 181.3 55.13) (width 0.2) (layer "F.Cu") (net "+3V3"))
 (segment (start 236.575 54.305) (end 182.125 54.305) (width 0.2) (layer "B.Cu") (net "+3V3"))
 (segment (start 182.125 54.305) (end 181.3 55.13) (width 0.2) (layer "B.Cu") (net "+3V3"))
 (segment (start 237.75 55.48) (end 236.575 54.305) (width 0.2) (layer "B.Cu") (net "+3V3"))
 (segment (start 201.654 101.797) (end 217.133 101.797) (width 0.2) (layer "F.Cu") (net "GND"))
 (segment (start 175.35 79.48) (end 179.5 83.63) (width 0.2) (layer "F.Cu") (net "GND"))
 (segment (start 175.975 53.955) (end 175.35 54.58) (width 0.2) (layer "F.Cu") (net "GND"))
 (segment (start 240.2 60.83) (end 233 60.83) (width 0.2) (layer "F.Cu") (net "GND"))
 (segment (start 223.8 95.13) (end 234.95 83.98) (width 0.2) (layer "F.Cu") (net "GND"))
 (segment (start 198.06 98.203) (end 201.654 101.797) (width 0.2) (layer "F.Cu") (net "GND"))
 (segment (start 182.475 53.955) (end 179.663299 53.955) (width 0.2) (layer "F.Cu") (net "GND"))
 (segment (start 179.375 85.555) (end 181.3 83.63) (width 0.2) (layer "F.Cu") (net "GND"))
 (segment (start 234.95 83.98) (end 235.3 83.98) (width 0.2) (layer "F.Cu") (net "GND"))
 (segment (start 223.8 95.13) (end 229.4 100.73) (width 0.2) (layer "F.Cu") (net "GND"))
 (segment (start 176 91.73) (end 176 91.53) (width 0.2) (layer "F.Cu") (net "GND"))
 (segment (start 240.2 60.83) (end 240.2 78.63) (width 0.2) (layer "F.Cu") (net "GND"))
 (segment (start 183.75 60.48) (end 183.75 55.23) (width 0.2) (layer "F.Cu") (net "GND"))
 (segment (start 183.75 55.23) (end 182.475 53.955) (width 0.2) (layer "F.Cu") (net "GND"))
 (segment (start 183.75 78.28) (end 183.75 55.23) (width 0.2) (layer "F.Cu") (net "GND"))
 (segment (start 180.4 96.13) (end 176 91.73) (width 0.2) (layer "F.Cu") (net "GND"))
 (segment (start 179.5 83.63) (end 181.3 83.63) (width 0.2) (layer "F.Cu") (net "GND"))
 (segment (start 237.75 83.98) (end 237.75 81.08) (width 0.2) (layer "F.Cu") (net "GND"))
 (segment (start 229.4 100.73) (end 231.3 100.73) (width 0.2) (layer "F.Cu") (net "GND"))
 (segment (start 179.663299 53.955) (end 179.375 54.243299) (width 0.2) (layer "F.Cu") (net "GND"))
 (segment (start 235.3 83.98) (end 235.3 83.33) (width 0.2) (layer "F.Cu") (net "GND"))
 (segment (start 180.4 99.23) (end 184.8 103.63) (width 0.2) (layer "F.Cu") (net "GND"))
 (segment (start 199.1435 101.150082) (end 199.1435 99.2865) (width 0.2) (layer "F.Cu") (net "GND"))
 (segment (start 175.35 91.08) (end 175.35 79.48) (width 0.2) (layer "F.Cu") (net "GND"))
 (segment (start 217.133 101.797) (end 223.8 95.13) (width 0.2) (layer "F.Cu") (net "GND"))
 (segment (start 233 60.83) (end 231.8 59.63) (width 0.2) (layer "F.Cu") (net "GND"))
 (segment (start 237.75 81.08) (end 240.2 78.63) (width 0.2) (layer "F.Cu") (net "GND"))
 (segment (start 180.4 96.13) (end 175.35 91.08) (width 0.2) (layer "F.Cu") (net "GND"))
 (segment (start 179.375 54.243299) (end 179.375 88.155) (width 0.2) (layer "F.Cu") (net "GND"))
 (segment (start 180.4 96.13) (end 180.4 99.23) (width 0.2) (layer "F.Cu") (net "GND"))
 (segment (start 175.35 54.58) (end 175.35 59.28) (width 0.2) (layer "F.Cu") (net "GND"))
 (segment (start 184.8 103.63) (end 196.663582 103.63) (width 0.2) (layer "F.Cu") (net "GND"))
 (segment (start 176 91.53) (end 179.375 88.155) (width 0.2) (layer "F.Cu") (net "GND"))
 (segment (start 199.1435 99.2865) (end 198.06 98.203) (width 0.2) (layer "F.Cu") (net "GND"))
 (segment (start 182.475 53.955) (end 175.975 53.955) (width 0.2) (layer "F.Cu") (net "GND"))
 (segment (start 235.3 83.33) (end 231.8 79.83) (width 0.2) (layer "F.Cu") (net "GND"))
 (segment (start 235.3 83.98) (end 237.75 83.98) (width 0.2) (layer "F.Cu") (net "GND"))
 (segment (start 196.663582 103.63) (end 199.1435 101.150082) (width 0.2) (layer "F.Cu") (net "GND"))
 (segment (start 179.375 88.155) (end 180.35 89.13) (width 0.2) (layer "F.Cu") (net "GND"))
 (segment (start 185.8 87.63) (end 186.775 88.605) (width 0.2) (layer "F.Cu") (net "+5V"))
 (segment (start 186.775 93.705) (end 185.85 94.63) (width 0.2) (layer "F.Cu") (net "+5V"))
 (segment (start 186.775 88.605) (end 186.775 93.705) (width 0.2) (layer "F.Cu") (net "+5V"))
 (segment (start 191.022 93.705) (end 198.06 100.743) (width 0.2) (layer "F.Cu") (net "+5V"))
 (segment (start 186.775 93.705) (end 191.022 93.705) (width 0.2) (layer "F.Cu") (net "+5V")))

